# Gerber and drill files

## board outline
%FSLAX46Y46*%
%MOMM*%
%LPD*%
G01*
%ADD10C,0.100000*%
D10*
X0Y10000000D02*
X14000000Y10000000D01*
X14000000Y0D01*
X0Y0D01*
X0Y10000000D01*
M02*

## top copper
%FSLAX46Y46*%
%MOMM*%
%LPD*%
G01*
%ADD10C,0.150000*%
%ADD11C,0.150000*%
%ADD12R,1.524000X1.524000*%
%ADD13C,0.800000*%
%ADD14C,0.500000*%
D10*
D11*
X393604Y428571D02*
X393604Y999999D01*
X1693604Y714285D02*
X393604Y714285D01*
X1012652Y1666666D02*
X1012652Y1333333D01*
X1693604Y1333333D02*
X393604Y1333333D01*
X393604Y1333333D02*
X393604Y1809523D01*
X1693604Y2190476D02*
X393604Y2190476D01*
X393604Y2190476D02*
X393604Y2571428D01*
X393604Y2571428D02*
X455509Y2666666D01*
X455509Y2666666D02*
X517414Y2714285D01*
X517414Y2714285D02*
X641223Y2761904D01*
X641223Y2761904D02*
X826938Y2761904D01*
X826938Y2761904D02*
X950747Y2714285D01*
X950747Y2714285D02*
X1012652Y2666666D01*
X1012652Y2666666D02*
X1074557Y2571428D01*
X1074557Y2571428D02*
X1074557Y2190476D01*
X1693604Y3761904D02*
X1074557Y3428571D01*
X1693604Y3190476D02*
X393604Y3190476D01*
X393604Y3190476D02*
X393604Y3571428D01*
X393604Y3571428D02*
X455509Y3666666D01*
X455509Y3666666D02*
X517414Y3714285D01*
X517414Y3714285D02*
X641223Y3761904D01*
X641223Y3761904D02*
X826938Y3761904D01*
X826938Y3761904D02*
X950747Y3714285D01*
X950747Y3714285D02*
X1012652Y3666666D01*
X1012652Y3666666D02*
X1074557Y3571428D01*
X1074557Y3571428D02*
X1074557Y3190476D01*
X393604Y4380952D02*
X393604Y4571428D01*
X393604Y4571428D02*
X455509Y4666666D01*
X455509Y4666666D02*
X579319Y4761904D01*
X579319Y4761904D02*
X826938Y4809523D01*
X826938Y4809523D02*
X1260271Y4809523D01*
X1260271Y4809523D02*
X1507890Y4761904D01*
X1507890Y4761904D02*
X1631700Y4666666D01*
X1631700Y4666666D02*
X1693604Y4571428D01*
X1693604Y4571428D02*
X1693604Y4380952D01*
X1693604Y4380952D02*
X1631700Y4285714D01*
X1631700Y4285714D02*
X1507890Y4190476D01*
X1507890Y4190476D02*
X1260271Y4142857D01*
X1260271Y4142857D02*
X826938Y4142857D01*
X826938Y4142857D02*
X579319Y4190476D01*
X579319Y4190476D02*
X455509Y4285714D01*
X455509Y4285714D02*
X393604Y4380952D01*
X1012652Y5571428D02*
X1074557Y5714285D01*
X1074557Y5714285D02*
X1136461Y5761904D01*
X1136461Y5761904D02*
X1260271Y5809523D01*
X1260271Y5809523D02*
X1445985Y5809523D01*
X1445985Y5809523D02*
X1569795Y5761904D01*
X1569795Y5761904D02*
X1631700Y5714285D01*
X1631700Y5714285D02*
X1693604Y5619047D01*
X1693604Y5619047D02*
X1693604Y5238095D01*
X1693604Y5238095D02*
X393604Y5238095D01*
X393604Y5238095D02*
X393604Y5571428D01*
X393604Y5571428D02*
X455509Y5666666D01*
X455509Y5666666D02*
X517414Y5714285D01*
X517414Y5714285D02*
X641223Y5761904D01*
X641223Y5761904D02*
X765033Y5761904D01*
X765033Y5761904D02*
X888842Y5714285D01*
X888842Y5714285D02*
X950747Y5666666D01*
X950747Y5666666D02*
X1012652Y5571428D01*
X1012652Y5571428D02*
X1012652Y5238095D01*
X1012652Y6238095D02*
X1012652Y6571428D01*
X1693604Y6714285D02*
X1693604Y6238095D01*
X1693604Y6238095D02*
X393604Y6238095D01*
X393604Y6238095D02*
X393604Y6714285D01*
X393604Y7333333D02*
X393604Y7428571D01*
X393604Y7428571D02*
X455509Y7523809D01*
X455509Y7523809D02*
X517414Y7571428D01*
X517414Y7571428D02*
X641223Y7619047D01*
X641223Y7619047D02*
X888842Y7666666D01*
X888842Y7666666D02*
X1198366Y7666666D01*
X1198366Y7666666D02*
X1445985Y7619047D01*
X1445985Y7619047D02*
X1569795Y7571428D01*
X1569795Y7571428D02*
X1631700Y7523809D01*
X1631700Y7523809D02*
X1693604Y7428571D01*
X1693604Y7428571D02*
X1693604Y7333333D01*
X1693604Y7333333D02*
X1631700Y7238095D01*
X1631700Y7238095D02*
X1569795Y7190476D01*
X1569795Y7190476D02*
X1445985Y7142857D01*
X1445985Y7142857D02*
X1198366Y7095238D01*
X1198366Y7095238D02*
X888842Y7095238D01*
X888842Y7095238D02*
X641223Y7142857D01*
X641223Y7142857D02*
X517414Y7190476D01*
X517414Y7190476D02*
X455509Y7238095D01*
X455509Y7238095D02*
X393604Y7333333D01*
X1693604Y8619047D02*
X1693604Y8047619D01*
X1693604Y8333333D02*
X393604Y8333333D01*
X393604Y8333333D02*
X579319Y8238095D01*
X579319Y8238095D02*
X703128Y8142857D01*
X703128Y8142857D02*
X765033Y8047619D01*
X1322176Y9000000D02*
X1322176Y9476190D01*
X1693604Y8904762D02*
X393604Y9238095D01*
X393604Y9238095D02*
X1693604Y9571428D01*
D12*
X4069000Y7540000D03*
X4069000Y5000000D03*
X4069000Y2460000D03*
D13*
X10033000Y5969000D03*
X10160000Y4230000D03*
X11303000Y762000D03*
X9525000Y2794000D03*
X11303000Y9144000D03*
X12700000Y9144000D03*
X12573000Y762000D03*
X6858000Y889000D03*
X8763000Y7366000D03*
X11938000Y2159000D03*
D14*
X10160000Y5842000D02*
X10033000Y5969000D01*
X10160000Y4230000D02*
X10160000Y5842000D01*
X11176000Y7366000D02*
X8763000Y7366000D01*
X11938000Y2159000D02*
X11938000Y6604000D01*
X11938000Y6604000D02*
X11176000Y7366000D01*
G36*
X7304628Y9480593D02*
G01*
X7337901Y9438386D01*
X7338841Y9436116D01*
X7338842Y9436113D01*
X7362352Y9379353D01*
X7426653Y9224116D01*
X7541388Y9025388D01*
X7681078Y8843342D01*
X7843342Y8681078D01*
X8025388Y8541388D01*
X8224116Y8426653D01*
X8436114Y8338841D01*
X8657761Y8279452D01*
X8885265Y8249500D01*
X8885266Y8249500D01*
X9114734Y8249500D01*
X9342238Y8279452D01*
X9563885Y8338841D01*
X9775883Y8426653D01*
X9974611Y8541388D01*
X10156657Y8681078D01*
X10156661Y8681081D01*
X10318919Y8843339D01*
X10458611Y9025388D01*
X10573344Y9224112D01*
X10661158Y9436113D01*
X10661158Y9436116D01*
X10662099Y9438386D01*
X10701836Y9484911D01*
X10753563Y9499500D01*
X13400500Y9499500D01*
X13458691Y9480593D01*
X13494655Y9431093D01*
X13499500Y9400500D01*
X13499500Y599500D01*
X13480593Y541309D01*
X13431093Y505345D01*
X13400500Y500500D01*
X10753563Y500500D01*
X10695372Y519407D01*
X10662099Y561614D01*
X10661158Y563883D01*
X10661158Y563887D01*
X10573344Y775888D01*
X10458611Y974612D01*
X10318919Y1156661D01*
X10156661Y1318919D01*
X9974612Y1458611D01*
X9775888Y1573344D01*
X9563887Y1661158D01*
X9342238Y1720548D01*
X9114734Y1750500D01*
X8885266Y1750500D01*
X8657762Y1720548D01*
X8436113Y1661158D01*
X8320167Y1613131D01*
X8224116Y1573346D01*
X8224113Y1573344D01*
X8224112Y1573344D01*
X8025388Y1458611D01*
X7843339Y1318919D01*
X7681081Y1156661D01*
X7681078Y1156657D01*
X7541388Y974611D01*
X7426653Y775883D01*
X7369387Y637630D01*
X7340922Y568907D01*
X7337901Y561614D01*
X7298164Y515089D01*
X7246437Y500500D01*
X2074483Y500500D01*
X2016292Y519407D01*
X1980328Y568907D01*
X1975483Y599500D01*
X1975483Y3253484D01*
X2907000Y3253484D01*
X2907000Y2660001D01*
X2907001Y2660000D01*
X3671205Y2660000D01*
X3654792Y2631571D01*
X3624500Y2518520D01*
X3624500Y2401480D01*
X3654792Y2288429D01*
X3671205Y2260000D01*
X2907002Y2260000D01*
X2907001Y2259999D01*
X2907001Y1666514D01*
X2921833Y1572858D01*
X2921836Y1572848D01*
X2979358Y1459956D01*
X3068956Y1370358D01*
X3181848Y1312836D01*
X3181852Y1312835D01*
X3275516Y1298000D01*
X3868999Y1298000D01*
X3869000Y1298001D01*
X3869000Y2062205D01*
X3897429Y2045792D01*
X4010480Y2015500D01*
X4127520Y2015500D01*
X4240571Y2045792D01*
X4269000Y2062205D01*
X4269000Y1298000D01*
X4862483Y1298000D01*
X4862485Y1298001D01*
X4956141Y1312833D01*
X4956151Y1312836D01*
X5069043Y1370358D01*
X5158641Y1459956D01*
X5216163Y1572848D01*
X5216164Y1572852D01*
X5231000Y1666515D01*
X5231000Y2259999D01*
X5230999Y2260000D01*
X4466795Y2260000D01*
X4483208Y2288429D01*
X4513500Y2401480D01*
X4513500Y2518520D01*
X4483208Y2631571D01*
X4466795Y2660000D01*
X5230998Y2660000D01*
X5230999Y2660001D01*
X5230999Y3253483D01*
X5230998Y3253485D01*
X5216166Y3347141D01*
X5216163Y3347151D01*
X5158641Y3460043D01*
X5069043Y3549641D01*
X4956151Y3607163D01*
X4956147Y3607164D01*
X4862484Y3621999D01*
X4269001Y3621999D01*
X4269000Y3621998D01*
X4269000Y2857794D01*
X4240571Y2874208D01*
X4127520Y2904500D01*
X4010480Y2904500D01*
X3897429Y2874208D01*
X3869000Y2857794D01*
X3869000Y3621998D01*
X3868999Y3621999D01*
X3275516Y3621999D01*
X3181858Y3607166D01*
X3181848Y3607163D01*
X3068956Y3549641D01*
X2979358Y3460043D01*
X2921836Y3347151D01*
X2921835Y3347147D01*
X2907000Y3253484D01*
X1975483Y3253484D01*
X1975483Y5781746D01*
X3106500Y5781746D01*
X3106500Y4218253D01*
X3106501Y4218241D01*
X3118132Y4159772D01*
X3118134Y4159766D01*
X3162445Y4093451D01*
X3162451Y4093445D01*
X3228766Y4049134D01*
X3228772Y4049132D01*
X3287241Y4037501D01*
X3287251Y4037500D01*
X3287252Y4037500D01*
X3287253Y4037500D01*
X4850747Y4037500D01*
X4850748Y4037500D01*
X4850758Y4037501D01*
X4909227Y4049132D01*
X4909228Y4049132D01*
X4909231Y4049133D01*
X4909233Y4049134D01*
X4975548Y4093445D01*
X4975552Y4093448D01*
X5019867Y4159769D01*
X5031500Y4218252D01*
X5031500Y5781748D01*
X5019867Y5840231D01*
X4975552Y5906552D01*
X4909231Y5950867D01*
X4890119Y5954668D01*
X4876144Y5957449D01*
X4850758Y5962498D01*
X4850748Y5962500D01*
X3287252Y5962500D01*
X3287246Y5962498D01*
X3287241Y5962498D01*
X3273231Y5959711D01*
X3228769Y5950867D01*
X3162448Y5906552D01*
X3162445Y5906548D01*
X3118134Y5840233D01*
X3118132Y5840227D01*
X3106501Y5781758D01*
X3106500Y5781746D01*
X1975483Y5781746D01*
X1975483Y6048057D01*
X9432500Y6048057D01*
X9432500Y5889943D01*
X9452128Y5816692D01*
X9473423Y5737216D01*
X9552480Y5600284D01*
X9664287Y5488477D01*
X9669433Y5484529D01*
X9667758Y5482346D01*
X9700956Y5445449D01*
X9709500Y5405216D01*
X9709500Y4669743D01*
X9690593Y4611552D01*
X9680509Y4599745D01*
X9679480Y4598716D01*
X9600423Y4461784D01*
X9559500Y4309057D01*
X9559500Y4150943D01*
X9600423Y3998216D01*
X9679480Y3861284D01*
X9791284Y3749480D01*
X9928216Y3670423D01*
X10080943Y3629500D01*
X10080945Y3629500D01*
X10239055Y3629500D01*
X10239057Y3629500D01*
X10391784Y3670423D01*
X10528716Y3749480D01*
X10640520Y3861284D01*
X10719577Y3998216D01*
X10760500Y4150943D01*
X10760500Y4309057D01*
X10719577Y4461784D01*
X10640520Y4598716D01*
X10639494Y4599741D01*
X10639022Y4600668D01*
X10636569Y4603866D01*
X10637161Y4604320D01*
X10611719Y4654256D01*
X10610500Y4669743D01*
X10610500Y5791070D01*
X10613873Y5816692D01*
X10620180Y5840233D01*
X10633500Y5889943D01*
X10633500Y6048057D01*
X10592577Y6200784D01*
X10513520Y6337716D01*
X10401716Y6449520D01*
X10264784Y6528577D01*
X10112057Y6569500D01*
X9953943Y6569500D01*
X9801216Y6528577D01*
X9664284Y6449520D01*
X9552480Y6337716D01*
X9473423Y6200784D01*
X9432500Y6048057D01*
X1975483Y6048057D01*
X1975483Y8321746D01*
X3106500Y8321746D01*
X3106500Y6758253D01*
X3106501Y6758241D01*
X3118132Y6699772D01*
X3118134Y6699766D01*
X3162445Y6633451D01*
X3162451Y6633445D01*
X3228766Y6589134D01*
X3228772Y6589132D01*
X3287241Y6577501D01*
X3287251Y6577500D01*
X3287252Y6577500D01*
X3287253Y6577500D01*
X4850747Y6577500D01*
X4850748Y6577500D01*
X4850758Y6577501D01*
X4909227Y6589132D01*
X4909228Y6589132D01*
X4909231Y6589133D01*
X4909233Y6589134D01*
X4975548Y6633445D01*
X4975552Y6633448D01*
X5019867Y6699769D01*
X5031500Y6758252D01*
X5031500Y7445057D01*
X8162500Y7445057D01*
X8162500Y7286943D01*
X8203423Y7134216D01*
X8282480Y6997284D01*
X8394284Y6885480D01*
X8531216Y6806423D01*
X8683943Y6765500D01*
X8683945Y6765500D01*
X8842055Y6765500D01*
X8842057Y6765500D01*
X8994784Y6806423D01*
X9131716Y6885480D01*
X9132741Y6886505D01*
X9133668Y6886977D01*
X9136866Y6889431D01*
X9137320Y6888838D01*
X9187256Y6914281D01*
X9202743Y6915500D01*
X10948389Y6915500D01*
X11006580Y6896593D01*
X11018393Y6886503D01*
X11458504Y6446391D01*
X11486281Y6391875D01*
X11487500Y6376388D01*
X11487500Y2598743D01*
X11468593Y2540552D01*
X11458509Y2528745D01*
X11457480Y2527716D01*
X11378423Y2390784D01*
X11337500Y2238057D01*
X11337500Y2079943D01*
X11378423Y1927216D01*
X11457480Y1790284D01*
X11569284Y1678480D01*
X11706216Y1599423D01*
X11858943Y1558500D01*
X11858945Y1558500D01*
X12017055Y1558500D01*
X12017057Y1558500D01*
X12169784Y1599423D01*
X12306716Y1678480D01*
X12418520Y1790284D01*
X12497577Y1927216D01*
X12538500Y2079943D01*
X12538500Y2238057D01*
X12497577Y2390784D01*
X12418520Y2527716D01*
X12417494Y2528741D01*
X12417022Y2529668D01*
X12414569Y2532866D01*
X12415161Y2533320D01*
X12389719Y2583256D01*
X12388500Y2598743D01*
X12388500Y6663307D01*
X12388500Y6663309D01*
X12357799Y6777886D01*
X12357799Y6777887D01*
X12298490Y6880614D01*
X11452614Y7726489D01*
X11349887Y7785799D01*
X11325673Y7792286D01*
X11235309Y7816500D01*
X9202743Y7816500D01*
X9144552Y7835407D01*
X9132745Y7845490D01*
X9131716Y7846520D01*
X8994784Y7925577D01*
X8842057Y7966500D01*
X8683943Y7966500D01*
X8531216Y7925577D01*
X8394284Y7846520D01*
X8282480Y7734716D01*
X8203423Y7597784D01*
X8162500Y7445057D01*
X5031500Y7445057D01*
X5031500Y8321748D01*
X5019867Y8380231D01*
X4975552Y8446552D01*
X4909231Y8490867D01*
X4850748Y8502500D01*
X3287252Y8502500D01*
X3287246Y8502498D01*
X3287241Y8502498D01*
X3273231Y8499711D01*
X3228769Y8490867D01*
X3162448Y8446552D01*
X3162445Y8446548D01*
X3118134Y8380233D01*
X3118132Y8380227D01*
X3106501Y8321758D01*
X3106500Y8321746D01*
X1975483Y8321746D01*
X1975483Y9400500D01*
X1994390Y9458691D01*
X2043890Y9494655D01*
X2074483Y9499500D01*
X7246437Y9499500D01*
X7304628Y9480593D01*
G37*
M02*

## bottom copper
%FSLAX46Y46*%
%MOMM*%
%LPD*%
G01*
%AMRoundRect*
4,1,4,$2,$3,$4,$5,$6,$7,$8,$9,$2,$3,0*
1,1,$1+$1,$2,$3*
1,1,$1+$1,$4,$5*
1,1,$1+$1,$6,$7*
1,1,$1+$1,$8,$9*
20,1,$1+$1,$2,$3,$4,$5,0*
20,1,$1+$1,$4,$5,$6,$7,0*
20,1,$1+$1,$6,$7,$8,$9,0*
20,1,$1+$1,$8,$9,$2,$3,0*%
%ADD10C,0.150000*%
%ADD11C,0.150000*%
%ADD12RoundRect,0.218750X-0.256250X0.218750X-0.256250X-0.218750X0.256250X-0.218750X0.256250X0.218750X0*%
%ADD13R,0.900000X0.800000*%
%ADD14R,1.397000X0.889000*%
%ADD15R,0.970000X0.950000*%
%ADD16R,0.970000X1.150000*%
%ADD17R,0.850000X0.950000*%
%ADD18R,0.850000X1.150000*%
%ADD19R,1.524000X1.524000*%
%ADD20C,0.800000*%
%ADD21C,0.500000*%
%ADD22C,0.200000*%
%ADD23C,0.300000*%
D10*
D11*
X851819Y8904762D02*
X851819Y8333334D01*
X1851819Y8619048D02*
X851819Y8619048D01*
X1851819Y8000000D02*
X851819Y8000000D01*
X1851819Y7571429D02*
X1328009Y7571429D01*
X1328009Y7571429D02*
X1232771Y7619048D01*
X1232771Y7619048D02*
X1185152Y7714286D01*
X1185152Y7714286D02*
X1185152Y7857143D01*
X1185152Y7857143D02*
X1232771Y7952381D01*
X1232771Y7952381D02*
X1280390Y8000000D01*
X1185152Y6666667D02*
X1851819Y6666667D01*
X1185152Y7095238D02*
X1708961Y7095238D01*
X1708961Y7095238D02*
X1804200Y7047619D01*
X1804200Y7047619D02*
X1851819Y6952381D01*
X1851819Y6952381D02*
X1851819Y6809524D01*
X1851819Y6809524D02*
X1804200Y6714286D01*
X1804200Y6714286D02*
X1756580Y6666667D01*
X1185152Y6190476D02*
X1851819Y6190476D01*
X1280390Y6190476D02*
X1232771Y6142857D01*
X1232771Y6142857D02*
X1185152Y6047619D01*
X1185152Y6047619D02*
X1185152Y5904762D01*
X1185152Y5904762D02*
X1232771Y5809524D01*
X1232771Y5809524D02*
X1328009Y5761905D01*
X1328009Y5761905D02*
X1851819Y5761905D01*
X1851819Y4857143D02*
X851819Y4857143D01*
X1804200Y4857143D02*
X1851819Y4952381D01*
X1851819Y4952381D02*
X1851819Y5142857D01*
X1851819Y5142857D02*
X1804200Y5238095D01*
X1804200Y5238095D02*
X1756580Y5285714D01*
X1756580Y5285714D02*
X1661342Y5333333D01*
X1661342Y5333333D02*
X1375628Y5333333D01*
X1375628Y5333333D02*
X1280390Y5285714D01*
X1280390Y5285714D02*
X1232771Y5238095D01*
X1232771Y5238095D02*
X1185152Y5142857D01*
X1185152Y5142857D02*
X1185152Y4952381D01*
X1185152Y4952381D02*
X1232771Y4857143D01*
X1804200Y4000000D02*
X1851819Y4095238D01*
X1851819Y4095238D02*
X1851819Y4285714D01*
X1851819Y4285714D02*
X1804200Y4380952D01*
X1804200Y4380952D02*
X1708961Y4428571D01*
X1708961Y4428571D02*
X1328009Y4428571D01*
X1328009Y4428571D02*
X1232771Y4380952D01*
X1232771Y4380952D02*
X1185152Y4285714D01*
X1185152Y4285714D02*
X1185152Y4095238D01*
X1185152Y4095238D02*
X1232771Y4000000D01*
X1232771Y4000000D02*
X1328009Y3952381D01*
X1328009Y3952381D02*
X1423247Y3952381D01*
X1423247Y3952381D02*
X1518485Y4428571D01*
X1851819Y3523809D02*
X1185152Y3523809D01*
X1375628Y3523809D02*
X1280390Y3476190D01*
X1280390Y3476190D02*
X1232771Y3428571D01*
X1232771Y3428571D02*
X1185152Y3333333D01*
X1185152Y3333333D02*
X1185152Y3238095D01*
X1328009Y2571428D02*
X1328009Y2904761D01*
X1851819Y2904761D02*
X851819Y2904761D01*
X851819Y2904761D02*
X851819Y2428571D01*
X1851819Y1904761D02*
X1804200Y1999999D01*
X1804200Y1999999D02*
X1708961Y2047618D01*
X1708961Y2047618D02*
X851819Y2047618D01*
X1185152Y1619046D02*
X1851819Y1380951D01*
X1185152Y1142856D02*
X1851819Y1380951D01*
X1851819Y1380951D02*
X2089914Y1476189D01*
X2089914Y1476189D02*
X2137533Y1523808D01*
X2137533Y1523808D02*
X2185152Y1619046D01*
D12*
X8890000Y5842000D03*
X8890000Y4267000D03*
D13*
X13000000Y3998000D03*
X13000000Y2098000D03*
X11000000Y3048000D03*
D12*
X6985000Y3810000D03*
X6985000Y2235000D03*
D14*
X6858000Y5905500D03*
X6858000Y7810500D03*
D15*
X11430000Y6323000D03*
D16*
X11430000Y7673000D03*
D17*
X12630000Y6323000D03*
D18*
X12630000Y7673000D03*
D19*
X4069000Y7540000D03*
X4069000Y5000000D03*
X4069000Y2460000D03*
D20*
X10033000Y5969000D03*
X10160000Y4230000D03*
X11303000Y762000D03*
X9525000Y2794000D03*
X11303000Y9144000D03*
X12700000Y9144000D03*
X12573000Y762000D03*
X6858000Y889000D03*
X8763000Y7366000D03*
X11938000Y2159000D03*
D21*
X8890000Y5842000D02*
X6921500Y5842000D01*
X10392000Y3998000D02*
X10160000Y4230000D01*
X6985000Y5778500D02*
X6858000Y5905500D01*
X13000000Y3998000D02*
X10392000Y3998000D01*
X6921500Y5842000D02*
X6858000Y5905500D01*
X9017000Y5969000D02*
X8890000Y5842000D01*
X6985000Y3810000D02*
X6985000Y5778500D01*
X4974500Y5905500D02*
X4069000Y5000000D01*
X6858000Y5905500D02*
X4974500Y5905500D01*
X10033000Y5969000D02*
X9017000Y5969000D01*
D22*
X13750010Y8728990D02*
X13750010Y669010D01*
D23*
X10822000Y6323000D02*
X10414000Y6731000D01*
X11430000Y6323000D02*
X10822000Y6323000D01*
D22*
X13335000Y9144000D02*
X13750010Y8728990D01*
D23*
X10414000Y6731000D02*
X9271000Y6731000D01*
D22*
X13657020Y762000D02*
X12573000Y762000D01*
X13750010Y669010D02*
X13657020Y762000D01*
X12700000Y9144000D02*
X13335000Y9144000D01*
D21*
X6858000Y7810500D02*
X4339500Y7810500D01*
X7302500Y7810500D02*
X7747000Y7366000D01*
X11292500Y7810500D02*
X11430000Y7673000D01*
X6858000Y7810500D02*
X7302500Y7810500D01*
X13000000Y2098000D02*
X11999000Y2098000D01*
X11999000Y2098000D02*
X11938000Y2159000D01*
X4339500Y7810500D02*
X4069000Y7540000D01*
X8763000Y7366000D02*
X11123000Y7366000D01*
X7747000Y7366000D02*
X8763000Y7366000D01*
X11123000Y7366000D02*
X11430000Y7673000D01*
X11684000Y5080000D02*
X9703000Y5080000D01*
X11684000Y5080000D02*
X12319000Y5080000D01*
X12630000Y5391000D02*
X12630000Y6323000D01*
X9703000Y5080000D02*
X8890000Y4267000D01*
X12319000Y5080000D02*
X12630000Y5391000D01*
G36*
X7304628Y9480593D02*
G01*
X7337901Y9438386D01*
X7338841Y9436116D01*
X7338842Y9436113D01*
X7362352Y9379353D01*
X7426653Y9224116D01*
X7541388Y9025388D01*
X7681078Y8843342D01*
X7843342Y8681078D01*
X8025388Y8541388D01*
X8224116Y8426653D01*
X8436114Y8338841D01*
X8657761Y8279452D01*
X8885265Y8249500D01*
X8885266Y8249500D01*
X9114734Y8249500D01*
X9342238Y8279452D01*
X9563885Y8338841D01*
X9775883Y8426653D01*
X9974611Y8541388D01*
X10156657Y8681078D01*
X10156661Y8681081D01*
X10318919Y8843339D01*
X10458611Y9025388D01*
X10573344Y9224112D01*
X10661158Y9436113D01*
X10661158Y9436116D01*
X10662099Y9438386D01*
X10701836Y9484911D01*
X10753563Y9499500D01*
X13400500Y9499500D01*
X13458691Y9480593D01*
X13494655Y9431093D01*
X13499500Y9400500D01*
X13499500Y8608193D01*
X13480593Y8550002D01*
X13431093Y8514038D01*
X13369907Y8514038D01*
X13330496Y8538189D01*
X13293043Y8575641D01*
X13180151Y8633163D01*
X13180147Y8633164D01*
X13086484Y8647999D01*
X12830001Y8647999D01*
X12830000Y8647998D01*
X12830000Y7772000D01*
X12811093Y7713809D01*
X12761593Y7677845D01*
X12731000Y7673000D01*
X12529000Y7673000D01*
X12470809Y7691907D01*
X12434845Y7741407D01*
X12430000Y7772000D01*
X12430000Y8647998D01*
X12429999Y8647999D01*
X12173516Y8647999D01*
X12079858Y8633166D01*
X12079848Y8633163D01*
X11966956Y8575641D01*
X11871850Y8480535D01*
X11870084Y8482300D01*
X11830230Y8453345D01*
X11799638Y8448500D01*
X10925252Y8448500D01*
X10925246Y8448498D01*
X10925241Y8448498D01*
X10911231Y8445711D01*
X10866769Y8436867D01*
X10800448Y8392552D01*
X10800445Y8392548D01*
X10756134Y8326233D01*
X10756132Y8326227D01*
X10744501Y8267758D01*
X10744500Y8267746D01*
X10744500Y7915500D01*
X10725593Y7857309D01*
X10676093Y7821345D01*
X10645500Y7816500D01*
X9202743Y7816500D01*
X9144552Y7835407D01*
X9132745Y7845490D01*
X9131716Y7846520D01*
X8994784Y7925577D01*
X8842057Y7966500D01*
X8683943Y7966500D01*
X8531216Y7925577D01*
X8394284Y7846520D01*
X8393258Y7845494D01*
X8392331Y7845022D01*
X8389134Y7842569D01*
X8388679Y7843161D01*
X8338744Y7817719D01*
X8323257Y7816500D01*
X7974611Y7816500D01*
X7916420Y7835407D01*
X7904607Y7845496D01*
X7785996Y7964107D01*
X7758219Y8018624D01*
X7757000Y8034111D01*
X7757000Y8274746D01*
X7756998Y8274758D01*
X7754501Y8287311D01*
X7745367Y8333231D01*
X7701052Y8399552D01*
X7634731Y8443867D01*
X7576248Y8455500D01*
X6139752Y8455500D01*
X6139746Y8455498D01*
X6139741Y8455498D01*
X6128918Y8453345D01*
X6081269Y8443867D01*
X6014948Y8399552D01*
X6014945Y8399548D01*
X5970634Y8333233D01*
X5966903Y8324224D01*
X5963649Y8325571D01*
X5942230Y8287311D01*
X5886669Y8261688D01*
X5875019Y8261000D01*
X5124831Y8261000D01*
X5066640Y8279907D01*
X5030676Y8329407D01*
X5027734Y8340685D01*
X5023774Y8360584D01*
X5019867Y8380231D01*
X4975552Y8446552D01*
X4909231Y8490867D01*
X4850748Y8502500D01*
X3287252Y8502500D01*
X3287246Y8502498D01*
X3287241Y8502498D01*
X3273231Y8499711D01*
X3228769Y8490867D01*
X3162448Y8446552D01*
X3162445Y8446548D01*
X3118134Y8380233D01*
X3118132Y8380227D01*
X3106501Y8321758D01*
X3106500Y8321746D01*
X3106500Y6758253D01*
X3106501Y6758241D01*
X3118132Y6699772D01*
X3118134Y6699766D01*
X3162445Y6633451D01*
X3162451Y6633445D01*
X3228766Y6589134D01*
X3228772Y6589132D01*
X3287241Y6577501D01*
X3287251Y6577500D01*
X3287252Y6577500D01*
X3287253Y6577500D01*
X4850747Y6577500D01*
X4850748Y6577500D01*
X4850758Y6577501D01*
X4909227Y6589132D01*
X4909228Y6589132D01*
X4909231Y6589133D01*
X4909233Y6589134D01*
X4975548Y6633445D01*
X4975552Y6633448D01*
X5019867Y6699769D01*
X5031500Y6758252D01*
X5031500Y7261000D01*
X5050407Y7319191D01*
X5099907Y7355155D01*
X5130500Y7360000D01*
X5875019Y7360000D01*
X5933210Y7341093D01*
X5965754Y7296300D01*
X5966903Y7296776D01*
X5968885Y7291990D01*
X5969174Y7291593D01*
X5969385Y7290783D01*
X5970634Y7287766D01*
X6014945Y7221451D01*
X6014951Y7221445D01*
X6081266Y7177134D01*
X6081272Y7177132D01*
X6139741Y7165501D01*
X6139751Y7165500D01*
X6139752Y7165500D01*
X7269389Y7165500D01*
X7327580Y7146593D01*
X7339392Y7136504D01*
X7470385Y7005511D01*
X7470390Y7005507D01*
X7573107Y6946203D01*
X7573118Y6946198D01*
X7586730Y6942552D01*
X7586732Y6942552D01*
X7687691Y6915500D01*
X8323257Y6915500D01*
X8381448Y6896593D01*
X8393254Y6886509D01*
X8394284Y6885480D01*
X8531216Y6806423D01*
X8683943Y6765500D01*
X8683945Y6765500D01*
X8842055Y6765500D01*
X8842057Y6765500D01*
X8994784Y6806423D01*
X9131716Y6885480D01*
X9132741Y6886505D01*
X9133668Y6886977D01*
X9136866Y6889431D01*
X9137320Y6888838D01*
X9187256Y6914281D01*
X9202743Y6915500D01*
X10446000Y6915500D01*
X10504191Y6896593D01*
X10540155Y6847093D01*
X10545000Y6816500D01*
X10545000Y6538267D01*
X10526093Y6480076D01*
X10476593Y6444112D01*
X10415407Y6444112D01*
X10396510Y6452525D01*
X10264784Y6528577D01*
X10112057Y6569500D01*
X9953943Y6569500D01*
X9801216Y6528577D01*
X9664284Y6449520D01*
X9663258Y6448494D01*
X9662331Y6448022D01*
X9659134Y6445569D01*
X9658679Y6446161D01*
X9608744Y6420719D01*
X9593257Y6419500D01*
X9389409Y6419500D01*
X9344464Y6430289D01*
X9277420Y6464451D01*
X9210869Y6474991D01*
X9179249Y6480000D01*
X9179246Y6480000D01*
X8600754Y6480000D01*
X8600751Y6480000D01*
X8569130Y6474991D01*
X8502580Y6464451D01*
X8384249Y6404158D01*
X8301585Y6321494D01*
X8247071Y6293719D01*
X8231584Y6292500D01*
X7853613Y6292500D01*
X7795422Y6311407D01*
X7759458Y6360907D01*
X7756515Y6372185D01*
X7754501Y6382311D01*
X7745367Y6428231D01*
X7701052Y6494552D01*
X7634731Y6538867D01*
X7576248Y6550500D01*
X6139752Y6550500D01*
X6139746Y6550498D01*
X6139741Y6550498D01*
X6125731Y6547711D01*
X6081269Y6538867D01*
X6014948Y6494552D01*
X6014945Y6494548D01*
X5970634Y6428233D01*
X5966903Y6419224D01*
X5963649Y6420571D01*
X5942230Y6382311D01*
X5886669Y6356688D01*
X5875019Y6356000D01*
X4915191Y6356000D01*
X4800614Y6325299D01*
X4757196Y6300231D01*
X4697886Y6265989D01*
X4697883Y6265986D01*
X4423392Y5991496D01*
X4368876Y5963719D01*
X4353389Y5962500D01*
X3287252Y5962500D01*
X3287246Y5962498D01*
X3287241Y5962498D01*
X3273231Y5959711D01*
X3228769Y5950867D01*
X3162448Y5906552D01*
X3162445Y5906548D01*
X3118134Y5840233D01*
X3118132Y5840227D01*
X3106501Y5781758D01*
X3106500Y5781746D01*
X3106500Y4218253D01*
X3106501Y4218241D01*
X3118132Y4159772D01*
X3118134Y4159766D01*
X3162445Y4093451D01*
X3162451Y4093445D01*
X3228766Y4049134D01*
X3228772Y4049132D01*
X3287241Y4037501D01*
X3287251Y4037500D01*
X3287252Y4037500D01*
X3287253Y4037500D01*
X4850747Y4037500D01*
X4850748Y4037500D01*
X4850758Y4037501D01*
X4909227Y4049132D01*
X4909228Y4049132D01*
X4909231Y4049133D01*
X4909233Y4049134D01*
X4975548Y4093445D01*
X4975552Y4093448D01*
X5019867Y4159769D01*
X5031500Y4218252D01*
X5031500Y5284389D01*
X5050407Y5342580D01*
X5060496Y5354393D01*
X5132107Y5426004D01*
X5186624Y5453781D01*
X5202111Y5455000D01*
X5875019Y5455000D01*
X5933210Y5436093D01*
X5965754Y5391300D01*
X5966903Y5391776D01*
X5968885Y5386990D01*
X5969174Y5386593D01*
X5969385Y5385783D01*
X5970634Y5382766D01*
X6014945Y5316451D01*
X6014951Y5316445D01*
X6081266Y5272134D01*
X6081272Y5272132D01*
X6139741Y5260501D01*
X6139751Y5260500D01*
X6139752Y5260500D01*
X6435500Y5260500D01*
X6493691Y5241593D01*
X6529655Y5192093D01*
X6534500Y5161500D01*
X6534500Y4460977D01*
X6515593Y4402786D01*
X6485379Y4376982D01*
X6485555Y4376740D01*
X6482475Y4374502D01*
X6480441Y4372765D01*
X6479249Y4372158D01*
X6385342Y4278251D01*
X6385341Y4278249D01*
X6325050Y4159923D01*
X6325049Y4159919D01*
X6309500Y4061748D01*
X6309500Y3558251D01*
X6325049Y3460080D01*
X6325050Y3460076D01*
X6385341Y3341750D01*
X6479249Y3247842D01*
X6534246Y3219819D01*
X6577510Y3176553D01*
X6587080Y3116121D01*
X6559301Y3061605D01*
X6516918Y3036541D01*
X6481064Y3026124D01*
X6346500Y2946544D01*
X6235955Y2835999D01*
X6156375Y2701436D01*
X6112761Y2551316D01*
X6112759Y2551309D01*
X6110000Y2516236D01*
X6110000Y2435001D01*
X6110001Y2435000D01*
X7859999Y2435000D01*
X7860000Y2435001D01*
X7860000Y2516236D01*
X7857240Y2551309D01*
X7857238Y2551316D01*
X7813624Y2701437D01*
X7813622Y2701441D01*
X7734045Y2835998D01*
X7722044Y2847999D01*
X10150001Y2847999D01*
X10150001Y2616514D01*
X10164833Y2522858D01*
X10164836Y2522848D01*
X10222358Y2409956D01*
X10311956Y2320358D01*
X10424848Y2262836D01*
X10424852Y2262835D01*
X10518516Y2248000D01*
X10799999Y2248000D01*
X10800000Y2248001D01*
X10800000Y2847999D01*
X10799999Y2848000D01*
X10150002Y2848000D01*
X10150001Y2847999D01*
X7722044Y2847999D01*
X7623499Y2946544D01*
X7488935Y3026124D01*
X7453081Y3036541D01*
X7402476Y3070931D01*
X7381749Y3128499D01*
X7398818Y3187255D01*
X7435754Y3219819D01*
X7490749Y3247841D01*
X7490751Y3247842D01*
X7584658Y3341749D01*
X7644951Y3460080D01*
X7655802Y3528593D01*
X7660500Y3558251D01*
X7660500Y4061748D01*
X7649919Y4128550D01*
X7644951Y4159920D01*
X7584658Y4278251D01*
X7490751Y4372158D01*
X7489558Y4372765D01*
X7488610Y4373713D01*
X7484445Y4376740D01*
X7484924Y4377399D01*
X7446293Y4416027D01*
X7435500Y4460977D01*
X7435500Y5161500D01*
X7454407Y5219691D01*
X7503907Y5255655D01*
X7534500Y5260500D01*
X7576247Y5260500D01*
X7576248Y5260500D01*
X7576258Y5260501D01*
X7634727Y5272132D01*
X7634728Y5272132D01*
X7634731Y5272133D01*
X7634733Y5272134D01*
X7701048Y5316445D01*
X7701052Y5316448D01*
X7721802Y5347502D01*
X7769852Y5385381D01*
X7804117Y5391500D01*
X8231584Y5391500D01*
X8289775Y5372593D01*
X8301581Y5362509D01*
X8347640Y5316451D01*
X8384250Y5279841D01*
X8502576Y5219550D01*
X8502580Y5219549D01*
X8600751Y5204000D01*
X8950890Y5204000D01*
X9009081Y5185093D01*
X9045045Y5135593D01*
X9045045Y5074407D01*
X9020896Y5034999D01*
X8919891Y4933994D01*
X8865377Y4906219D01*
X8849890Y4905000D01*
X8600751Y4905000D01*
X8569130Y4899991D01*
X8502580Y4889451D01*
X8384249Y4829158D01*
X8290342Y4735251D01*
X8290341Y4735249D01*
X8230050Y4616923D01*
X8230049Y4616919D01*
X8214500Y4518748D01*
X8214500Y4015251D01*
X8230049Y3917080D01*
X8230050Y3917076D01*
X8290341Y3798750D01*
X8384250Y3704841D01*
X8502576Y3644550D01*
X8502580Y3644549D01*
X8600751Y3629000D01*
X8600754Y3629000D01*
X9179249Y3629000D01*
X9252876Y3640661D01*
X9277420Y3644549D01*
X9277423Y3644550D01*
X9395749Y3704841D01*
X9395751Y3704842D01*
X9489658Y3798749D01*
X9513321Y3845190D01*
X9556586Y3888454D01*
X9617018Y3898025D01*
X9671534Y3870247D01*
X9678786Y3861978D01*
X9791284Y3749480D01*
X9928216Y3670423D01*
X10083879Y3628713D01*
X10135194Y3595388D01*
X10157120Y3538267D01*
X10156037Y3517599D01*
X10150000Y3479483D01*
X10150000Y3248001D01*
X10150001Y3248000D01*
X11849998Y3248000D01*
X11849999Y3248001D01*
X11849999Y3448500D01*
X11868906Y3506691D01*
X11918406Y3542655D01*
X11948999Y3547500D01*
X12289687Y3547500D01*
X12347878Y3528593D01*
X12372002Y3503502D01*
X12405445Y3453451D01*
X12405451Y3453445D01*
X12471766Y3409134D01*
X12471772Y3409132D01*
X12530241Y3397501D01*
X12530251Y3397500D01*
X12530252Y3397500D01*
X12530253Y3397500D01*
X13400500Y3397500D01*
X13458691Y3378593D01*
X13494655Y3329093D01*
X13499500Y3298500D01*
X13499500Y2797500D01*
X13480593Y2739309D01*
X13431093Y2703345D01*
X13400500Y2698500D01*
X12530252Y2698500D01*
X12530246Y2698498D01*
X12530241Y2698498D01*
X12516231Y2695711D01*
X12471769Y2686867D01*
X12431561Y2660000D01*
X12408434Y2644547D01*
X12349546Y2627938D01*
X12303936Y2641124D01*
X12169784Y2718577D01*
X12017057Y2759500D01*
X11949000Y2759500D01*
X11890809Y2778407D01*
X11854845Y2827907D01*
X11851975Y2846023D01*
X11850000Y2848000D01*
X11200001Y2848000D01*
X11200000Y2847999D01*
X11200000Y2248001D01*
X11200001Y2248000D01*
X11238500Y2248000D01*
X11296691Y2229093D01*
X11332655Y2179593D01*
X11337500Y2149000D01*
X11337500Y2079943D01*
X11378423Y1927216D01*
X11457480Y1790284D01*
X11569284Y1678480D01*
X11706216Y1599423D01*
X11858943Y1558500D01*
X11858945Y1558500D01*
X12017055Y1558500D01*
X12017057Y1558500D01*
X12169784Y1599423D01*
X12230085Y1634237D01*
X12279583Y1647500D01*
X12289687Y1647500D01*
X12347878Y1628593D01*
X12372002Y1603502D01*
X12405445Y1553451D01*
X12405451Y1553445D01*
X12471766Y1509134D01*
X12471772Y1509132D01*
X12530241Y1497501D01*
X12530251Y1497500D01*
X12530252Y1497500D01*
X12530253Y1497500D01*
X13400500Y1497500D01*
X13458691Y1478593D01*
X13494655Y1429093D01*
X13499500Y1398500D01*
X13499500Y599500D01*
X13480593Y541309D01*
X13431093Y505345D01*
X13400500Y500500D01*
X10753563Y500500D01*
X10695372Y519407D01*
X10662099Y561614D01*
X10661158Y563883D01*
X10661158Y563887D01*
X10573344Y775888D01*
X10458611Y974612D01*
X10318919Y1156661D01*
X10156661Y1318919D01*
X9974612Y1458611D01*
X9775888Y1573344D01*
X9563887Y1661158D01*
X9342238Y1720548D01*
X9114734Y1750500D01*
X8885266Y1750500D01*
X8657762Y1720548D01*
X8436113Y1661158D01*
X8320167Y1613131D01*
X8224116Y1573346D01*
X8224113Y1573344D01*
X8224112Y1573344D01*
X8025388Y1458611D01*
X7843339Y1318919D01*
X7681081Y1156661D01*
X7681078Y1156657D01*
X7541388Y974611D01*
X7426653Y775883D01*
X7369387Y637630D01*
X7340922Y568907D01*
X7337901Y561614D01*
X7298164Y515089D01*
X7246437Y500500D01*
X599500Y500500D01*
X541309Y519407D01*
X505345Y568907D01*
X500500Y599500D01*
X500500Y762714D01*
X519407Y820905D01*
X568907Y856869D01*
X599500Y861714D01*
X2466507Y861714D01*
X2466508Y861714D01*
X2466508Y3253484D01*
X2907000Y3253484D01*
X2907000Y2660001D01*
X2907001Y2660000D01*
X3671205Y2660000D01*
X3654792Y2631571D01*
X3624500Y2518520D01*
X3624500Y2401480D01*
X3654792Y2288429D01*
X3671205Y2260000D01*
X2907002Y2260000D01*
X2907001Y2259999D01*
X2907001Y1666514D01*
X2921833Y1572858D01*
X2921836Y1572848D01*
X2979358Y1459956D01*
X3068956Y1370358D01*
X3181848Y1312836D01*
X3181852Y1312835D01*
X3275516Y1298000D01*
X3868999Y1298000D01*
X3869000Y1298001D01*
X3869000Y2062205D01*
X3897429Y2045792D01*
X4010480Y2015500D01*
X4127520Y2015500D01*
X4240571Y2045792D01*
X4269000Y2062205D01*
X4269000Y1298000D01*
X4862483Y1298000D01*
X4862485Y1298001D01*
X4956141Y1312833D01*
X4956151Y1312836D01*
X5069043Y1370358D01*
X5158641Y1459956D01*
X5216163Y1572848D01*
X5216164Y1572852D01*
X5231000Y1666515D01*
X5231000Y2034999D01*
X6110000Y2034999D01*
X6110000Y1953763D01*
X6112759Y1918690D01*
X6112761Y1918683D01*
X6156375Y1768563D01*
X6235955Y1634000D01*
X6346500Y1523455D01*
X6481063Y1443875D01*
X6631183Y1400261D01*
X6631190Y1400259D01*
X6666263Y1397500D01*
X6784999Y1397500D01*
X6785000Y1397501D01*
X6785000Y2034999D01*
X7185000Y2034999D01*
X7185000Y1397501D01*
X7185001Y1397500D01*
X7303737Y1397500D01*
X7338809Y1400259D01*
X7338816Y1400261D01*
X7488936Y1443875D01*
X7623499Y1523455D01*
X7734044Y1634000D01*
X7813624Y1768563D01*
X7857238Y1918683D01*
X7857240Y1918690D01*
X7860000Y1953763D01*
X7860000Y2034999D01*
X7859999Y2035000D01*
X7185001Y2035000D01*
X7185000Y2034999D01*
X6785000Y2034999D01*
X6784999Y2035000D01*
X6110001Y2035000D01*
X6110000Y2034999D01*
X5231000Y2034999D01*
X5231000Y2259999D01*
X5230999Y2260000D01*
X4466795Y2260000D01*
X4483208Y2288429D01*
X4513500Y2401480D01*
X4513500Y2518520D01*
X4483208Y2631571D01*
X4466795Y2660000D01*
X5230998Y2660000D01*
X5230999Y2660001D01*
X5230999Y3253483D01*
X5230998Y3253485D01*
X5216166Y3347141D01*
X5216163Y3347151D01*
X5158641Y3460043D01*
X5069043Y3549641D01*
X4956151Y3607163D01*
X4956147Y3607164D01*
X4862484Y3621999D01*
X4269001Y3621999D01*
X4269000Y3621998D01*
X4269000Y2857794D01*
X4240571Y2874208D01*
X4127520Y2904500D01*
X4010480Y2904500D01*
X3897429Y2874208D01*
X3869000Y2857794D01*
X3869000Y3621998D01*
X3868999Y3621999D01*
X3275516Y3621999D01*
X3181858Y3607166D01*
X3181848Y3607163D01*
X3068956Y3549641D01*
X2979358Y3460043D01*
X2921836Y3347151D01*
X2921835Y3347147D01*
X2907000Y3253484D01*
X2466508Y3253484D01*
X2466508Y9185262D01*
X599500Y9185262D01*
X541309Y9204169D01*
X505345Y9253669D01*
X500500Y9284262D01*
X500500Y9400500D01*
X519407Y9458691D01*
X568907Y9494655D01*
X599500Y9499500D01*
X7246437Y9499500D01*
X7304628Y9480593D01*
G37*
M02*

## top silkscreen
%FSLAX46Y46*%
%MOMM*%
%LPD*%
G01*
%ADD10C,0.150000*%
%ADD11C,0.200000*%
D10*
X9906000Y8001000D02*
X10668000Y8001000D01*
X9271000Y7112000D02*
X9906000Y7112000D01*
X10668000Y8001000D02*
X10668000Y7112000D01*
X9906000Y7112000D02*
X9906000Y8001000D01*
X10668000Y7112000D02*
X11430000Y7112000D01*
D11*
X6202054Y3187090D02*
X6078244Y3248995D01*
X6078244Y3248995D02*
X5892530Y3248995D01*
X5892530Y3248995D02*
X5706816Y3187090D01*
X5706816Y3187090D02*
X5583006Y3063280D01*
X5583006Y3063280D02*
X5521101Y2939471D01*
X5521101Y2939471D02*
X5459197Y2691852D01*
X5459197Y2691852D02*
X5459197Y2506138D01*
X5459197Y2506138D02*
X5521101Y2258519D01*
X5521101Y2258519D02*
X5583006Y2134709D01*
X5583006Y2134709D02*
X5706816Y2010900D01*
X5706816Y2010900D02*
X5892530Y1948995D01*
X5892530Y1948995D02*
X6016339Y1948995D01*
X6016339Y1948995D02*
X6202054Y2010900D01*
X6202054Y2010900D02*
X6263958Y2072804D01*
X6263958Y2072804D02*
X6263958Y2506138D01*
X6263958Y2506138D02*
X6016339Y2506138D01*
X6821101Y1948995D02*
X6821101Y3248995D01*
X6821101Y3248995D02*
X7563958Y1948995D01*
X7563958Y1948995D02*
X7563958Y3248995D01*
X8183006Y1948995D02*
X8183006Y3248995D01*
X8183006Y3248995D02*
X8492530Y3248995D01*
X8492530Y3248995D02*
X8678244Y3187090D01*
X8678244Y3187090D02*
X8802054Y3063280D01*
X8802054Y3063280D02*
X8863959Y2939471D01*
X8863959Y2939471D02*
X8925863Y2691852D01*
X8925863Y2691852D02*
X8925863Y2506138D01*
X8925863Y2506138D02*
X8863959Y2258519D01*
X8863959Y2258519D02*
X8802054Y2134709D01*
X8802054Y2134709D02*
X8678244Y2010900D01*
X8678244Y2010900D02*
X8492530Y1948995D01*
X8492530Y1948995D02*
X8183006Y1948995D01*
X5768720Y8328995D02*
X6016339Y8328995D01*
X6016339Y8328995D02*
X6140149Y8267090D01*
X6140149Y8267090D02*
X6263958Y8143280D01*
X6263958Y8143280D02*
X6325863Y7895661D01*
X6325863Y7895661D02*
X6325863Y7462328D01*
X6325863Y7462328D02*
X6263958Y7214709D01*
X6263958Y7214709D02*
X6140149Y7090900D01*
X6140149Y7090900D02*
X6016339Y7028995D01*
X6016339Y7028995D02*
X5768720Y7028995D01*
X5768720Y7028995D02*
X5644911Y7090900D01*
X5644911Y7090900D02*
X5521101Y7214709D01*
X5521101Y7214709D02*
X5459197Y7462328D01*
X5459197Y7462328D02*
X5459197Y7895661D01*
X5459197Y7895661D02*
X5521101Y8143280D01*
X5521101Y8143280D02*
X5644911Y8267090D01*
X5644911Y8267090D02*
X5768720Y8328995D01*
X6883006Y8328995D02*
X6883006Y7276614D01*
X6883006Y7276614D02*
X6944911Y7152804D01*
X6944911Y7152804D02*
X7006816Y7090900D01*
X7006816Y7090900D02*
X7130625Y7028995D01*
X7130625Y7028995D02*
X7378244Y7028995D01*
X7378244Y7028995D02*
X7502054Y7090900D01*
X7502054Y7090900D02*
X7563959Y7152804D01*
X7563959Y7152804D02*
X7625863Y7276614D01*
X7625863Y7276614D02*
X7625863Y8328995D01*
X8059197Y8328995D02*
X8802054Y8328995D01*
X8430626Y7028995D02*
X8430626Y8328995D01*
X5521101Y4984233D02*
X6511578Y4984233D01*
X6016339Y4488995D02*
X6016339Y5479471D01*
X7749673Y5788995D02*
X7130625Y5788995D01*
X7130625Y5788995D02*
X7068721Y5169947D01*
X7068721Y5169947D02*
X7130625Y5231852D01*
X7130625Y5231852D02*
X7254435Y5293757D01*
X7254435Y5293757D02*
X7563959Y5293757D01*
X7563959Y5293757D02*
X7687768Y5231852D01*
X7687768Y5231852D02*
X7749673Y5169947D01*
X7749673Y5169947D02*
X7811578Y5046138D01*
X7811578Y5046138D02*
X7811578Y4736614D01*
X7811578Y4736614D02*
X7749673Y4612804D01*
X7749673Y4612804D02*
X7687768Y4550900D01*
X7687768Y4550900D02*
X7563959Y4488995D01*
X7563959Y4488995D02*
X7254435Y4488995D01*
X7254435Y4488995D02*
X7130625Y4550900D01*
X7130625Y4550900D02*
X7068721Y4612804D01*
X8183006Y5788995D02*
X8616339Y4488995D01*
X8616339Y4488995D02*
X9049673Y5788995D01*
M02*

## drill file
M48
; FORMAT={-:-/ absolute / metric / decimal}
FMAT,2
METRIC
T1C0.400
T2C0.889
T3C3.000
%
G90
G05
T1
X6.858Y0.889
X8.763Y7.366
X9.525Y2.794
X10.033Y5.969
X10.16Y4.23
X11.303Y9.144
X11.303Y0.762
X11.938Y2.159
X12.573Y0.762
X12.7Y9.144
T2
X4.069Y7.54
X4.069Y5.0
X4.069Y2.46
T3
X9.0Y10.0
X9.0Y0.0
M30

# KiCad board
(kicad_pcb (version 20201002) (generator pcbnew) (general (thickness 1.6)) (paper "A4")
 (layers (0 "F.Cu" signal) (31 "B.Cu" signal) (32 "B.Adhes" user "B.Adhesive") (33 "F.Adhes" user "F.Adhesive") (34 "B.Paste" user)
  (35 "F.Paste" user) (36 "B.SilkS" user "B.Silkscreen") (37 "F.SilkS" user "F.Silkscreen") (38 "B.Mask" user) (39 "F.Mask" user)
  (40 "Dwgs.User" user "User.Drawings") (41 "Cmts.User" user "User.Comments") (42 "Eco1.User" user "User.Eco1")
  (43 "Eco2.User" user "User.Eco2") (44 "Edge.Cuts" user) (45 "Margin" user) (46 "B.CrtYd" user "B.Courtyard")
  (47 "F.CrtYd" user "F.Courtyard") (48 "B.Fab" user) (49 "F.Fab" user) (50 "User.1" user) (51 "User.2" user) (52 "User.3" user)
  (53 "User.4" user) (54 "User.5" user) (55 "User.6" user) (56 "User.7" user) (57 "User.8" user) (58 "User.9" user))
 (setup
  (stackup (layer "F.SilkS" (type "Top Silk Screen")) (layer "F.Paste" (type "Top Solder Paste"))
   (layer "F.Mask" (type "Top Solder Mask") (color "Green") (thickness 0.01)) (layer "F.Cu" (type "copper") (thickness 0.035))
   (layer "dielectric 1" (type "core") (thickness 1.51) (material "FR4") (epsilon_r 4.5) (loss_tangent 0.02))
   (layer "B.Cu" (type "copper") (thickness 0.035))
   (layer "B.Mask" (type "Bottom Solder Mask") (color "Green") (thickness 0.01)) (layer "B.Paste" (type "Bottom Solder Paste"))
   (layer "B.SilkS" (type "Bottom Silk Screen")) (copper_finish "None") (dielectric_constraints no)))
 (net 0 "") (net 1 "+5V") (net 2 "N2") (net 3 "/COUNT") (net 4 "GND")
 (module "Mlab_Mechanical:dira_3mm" (layer "F.Cu") (at 8.89 -10.033)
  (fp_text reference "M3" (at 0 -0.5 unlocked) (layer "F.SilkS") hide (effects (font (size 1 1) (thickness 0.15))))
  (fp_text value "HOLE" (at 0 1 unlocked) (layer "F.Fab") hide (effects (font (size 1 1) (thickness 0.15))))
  (pad "" np_thru_hole circle (at 0.11 0.033) (size 3 3) (drill 3) (layers *.Mask)))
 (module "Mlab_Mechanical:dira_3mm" (layer "F.Cu") (at 9 0)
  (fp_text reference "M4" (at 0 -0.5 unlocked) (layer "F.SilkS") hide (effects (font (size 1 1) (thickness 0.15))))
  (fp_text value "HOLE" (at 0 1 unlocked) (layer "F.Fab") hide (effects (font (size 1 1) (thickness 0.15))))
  (pad "" np_thru_hole circle (at 0 0) (size 3 3) (drill 3) (layers *.Mask)))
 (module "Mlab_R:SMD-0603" (layer "B.Cu") (at 8.89 -5.0545 -90)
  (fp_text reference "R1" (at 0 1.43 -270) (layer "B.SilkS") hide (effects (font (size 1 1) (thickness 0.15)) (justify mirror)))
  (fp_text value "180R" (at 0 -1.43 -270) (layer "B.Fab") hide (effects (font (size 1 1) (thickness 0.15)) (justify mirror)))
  (pad "1" smd roundrect (at -0.7875 0 270) (size 0.875 0.95) (layers "B.Cu" "B.Paste" "B.Mask") (roundrect_rratio 0.25) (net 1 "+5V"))
  (pad "2" smd roundrect (at 0.7875 0 270) (size 0.875 0.95) (layers "B.Cu" "B.Paste" "B.Mask") (roundrect_rratio 0.25) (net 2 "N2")))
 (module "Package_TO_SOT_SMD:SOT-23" (layer "B.Cu") (at 12 -3.048 180)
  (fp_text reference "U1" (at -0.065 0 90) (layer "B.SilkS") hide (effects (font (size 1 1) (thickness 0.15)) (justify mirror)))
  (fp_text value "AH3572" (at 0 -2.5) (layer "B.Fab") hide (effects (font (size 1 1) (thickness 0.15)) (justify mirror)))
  (pad "1" smd rect (at -1 0.95 180) (size 0.9 0.8) (layers "B.Cu" "B.Paste" "B.Mask") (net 1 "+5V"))
  (pad "2" smd rect (at -1 -0.95 180) (size 0.9 0.8) (layers "B.Cu" "B.Paste" "B.Mask") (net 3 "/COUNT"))
  (pad "3" smd rect (at 1 0 180) (size 0.9 0.8) (layers "B.Cu" "B.Paste" "B.Mask") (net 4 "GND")))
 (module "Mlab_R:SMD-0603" (layer "B.Cu") (at 6.985 -3.0225 -90)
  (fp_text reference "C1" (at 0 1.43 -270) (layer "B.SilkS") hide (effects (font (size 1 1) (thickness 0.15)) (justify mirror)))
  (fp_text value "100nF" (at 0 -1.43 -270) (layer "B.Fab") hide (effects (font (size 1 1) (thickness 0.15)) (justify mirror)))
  (pad "1" smd roundrect (at -0.7875 0 270) (size 0.875 0.95) (layers "B.Cu" "B.Paste" "B.Mask") (roundrect_rratio 0.25) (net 1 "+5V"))
  (pad "2" smd roundrect (at 0.7875 0 270) (size 0.875 0.95) (layers "B.Cu" "B.Paste" "B.Mask") (roundrect_rratio 0.25) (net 4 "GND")))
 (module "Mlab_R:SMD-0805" (layer "B.Cu") (at 6.858 -6.858 90)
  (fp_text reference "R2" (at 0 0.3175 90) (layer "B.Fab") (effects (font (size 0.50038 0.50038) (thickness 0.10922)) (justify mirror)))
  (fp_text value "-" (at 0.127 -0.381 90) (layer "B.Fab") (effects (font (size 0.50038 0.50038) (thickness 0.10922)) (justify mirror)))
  (pad "1" smd rect (at -0.9525 0 90) (size 0.889 1.397) (layers "B.Cu" "B.Paste" "B.Mask") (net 1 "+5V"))
  (pad "2" smd rect (at 0.9525 0 90) (size 0.889 1.397) (layers "B.Cu" "B.Paste" "B.Mask") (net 3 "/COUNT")))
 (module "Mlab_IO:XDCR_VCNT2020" (layer "B.Cu") (at 12 -7.048)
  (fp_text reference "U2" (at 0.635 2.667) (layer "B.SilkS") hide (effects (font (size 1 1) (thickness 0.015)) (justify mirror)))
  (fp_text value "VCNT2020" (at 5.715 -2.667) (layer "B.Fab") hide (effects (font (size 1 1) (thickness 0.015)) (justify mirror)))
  (pad "1" smd rect (at -0.57 0.725) (size 0.97 0.95) (layers "B.Cu" "B.Paste" "B.Mask") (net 4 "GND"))
  (pad "2" smd rect (at -0.57 -0.625) (size 0.97 1.15) (layers "B.Cu" "B.Paste" "B.Mask") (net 3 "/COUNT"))
  (pad "3" smd rect (at 0.63 0.725) (size 0.85 0.95) (layers "B.Cu" "B.Paste" "B.Mask") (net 2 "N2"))
  (pad "4" smd rect (at 0.63 -0.625) (size 0.85 1.15) (layers "B.Cu" "B.Paste" "B.Mask") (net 4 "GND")))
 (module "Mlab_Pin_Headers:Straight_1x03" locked (layer "B.Cu") (at 4.069 -5 180)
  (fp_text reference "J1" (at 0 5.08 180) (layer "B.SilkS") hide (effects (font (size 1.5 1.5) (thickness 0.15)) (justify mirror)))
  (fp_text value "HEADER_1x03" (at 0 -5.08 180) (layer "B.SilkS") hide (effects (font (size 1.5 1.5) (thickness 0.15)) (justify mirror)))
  (pad "1" thru_hole rect (at 0 2.54 180) (size 1.524 1.524) (drill 0.889) (layers *.Cu *.Mask) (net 3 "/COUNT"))
  (pad "2" thru_hole rect (at 0 0 180) (size 1.524 1.524) (drill 0.889) (layers *.Cu *.Mask) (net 1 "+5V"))
  (pad "3" thru_hole rect (at 0 -2.54 180) (size 1.524 1.524) (drill 0.889) (layers *.Cu *.Mask) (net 4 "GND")))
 (gr_line (start 9.906 -8.001) (end 10.668 -8.001) (layer "F.SilkS") (width 0.15))
 (gr_line (start 9.271 -7.112) (end 9.906 -7.112) (layer "F.SilkS") (width 0.15))
 (gr_line (start 10.668 -8.001) (end 10.668 -7.112) (layer "F.SilkS") (width 0.15))
 (gr_line (start 9.906 -7.112) (end 9.906 -8.001) (layer "F.SilkS") (width 0.15))
 (gr_line (start 10.668 -7.112) (end 11.43 -7.112) (layer "F.SilkS") (width 0.15))
 (gr_rect (start 0 0) (end 14 -10) (layer "Edge.Cuts") (width 0.1))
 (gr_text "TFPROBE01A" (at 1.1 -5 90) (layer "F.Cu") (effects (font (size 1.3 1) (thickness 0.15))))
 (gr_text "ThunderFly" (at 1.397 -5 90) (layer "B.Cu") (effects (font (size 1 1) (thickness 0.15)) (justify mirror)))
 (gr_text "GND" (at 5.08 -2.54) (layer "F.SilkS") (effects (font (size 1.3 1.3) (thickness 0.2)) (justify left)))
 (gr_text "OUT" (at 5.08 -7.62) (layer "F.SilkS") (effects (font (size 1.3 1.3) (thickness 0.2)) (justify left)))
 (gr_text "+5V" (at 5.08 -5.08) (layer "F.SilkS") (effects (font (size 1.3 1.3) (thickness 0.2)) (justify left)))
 (segment (start 10.16 -5.842) (end 10.033 -5.969) (width 0.5) (layer "F.Cu") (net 1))
 (segment (start 10.16 -4.23) (end 10.16 -5.842) (width 0.5) (layer "F.Cu") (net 1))
 (via (at 10.033 -5.969) (size 0.8) (drill 0.4) (layers "F.Cu" "B.Cu") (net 1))
 (via (at 10.16 -4.23) (size 0.8) (drill 0.4) (layers "F.Cu" "B.Cu") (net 1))
 (segment (start 8.89 -5.842) (end 6.9215 -5.842) (width 0.5) (layer "B.Cu") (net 1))
 (segment (start 10.392 -3.998) (end 10.16 -4.23) (width 0.5) (layer "B.Cu") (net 1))
 (segment (start 6.985 -5.7785) (end 6.858 -5.9055) (width 0.5) (layer "B.Cu") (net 1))
 (segment (start 13 -3.998) (end 10.392 -3.998) (width 0.5) (layer "B.Cu") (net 1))
 (segment (start 6.9215 -5.842) (end 6.858 -5.9055) (width 0.5) (layer "B.Cu") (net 1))
 (segment (start 9.017 -5.969) (end 8.89 -5.842) (width 0.5) (layer "B.Cu") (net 1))
 (segment (start 6.985 -3.81) (end 6.985 -5.7785) (width 0.5) (layer "B.Cu") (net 1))
 (segment (start 4.9745 -5.9055) (end 4.069 -5) (width 0.5) (layer "B.Cu") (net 1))
 (segment (start 6.858 -5.9055) (end 4.9745 -5.9055) (width 0.5) (layer "B.Cu") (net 1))
 (segment (start 10.033 -5.969) (end 9.017 -5.969) (width 0.5) (layer "B.Cu") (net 1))
 (via (at 11.303 -0.762) (size 0.8) (drill 0.4) (layers "F.Cu" "B.Cu") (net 4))
 (via (at 9.525 -2.794) (size 0.8) (drill 0.4) (layers "F.Cu" "B.Cu") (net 4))
 (via (at 11.303 -9.144) (size 0.8) (drill 0.4) (layers "F.Cu" "B.Cu") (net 4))
 (via (at 12.7 -9.144) (size 0.8) (drill 0.4) (layers "F.Cu" "B.Cu") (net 4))
 (via (at 12.573 -0.762) (size 0.8) (drill 0.4) (layers "F.Cu" "B.Cu") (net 4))
 (via (at 6.858 -0.889) (size 0.8) (drill 0.4) (layers "F.Cu" "B.Cu") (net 4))
 (segment (start 13.75001 -8.72899) (end 13.75001 -0.66901) (width 0.2) (layer "B.Cu") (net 4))
 (segment (start 10.822 -6.323) (end 10.414 -6.731) (width 0.3) (layer "B.Cu") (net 4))
 (segment (start 11.43 -6.323) (end 10.822 -6.323) (width 0.3) (layer "B.Cu") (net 4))
 (segment (start 13.335 -9.144) (end 13.75001 -8.72899) (width 0.2) (layer "B.Cu") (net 4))
 (segment (start 10.414 -6.731) (end 9.271 -6.731) (width 0.3) (layer "B.Cu") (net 4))
 (segment (start 13.65702 -0.762) (end 12.573 -0.762) (width 0.2) (layer "B.Cu") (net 4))
 (segment (start 13.75001 -0.66901) (end 13.65702 -0.762) (width 0.2) (layer "B.Cu") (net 4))
 (segment (start 12.7 -9.144) (end 13.335 -9.144) (width 0.2) (layer "B.Cu") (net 4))
 (segment (start 11.176 -7.366) (end 8.763 -7.366) (width 0.5) (layer "F.Cu") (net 3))
 (segment (start 11.938 -2.159) (end 11.938 -6.604) (width 0.5) (layer "F.Cu") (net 3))
 (segment (start 11.938 -6.604) (end 11.176 -7.366) (width 0.5) (layer "F.Cu") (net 3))
 (via (at 8.763 -7.366) (size 0.8) (drill 0.4) (layers "F.Cu" "B.Cu") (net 3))
 (via (at 11.938 -2.159) (size 0.8) (drill 0.4) (layers "F.Cu" "B.Cu") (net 3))
 (segment (start 6.858 -7.8105) (end 4.3395 -7.8105) (width 0.5) (layer "B.Cu") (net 3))
 (segment (start 7.3025 -7.8105) (end 7.747 -7.366) (width 0.5) (layer "B.Cu") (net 3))
 (segment (start 11.2925 -7.8105) (end 11.43 -7.673) (width 0.5) (layer "B.Cu") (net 3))
 (segment (start 6.858 -7.8105) (end 7.3025 -7.8105) (width 0.5) (layer "B.Cu") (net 3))
 (segment (start 13 -2.098) (end 11.999 -2.098) (width 0.5) (layer "B.Cu") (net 3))
 (segment (start 11.999 -2.098) (end 11.938 -2.159) (width 0.5) (layer "B.Cu") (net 3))
 (segment (start 4.3395 -7.8105) (end 4.069 -7.54) (width 0.5) (layer "B.Cu") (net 3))
 (segment (start 8.763 -7.366) (end 11.123 -7.366) (width 0.5) (layer "B.Cu") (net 3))
 (segment (start 7.747 -7.366) (end 8.763 -7.366) (width 0.5) (layer "B.Cu") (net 3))
 (segment (start 11.123 -7.366) (end 11.43 -7.673) (width 0.5) (layer "B.Cu") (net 3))
 (segment (start 11.684 -5.08) (end 9.703 -5.08) (width 0.5) (layer "B.Cu") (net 2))
 (segment (start 11.684 -5.08) (end 12.319 -5.08) (width 0.5) (layer "B.Cu") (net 2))
 (segment (start 12.63 -5.391) (end 12.63 -6.323) (width 0.5) (layer "B.Cu") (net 2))
 (segment (start 9.703 -5.08) (end 8.89 -4.267) (width 0.5) (layer "B.Cu") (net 2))
 (segment (start 12.319 -5.08) (end 12.63 -5.391) (width 0.5) (layer "B.Cu") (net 2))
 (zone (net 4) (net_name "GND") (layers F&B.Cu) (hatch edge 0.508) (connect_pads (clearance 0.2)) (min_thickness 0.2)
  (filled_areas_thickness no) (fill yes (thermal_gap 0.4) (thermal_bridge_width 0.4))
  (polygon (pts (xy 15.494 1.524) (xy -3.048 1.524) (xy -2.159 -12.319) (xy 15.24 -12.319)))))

